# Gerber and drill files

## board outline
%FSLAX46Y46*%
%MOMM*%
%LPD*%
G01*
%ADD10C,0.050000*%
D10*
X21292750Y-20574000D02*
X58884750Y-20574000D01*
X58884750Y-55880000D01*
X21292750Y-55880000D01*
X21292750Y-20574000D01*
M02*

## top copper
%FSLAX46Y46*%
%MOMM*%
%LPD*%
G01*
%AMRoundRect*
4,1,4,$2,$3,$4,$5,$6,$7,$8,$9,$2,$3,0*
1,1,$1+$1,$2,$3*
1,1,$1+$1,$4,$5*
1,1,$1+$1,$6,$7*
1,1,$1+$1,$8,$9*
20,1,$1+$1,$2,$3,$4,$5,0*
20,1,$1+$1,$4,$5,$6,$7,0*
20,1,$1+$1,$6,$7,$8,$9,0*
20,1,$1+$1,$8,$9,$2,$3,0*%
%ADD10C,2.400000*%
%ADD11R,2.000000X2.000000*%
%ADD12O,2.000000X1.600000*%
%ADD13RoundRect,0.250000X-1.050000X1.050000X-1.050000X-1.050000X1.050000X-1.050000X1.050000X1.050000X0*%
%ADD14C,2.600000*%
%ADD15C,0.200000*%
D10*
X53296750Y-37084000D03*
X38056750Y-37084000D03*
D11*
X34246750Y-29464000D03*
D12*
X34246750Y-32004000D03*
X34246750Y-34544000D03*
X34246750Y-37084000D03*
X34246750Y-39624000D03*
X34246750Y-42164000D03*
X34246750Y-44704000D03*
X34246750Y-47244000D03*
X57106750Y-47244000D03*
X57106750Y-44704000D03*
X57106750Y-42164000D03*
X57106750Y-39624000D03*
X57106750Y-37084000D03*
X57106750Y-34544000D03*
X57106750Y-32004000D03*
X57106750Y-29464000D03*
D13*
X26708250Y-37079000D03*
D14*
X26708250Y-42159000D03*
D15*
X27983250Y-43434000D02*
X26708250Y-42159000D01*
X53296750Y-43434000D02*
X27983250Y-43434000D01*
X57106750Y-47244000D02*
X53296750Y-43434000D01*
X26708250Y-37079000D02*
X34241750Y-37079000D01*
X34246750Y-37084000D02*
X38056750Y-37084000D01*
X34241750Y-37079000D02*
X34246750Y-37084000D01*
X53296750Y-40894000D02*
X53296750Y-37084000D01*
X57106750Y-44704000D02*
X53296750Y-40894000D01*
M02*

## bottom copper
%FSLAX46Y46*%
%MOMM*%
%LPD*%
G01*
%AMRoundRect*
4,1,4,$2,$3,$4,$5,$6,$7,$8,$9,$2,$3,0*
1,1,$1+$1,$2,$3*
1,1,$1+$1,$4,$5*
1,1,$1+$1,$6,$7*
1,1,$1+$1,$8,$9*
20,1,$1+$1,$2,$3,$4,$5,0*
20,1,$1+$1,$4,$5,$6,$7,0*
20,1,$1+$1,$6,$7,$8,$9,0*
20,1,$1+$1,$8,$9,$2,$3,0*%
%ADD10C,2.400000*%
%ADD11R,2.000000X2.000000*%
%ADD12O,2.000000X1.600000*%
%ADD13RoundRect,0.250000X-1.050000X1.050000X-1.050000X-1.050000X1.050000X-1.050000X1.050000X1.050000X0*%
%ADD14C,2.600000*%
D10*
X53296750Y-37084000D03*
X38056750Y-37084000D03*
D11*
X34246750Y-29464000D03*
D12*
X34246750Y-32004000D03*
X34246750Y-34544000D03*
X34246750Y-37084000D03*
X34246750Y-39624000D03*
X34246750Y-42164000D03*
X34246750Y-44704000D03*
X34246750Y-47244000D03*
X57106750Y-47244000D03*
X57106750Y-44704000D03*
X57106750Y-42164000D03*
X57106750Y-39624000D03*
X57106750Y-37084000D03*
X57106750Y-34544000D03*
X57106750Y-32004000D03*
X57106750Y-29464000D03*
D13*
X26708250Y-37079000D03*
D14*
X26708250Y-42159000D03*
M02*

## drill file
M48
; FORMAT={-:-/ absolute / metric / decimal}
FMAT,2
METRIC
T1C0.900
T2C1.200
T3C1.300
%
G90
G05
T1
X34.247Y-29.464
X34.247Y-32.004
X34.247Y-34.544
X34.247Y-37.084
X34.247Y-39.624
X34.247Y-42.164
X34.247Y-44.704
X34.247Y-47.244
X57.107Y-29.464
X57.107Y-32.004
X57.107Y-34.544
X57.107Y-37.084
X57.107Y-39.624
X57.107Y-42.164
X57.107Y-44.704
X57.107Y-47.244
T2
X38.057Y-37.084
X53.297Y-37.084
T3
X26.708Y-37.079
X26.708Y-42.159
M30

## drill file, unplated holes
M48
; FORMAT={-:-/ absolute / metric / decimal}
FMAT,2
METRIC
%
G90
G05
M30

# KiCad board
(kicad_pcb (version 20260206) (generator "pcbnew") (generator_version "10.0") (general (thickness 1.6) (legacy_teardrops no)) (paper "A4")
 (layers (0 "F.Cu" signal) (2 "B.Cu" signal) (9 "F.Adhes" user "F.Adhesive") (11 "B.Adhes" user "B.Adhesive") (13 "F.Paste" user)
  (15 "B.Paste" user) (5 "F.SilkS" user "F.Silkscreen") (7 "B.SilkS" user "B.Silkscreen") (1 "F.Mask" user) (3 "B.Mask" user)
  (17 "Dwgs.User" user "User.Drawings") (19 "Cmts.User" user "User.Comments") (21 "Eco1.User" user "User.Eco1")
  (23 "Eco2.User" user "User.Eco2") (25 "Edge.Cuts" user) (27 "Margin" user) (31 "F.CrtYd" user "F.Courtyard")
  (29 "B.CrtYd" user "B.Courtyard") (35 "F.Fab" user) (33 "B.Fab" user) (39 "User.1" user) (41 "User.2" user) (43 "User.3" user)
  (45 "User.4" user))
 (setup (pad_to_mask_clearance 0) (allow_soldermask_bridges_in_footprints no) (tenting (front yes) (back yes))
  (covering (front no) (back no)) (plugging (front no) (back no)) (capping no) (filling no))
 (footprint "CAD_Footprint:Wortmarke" (layer "F.Cu") (at 26.924 47.498)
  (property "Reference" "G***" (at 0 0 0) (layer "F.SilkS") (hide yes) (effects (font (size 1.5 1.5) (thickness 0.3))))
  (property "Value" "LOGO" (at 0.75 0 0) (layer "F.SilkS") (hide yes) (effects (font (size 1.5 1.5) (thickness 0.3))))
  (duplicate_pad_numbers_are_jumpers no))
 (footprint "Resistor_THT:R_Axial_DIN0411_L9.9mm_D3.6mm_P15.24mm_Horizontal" (layer "F.Cu") (at 53.29675 37.084 180)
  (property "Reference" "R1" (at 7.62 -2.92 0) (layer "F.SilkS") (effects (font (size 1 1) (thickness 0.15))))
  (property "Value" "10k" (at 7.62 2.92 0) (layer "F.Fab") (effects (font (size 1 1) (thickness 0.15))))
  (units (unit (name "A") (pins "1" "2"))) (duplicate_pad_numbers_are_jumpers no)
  (pad "1" thru_hole circle (at 0 0 180) (size 2.4 2.4) (drill 1.2) (layers "*.Cu" "*.Mask") (remove_unused_layers no) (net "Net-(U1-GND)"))
  (pad "2" thru_hole circle (at 15.24 0 180) (size 2.4 2.4) (drill 1.2) (layers "*.Cu" "*.Mask") (remove_unused_layers no)
   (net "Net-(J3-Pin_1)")))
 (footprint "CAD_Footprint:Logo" (layer "F.Cu") (at 26.924 27.432)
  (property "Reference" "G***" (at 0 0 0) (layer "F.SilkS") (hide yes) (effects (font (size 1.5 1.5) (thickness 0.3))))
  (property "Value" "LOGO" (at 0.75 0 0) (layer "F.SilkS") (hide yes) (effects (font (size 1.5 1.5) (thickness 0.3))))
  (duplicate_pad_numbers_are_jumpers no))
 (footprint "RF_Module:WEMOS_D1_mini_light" (layer "F.Cu") (at 34.24675 29.464)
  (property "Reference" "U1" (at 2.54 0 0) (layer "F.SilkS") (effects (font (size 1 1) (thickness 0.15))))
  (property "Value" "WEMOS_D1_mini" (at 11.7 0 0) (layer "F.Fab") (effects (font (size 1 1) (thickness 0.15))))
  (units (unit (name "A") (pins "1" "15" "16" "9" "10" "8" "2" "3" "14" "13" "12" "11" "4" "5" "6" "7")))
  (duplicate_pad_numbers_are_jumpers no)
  (pad "1" thru_hole rect (at 0 0) (size 2 2) (drill 0.9) (layers "*.Cu" "*.Mask") (remove_unused_layers no)
   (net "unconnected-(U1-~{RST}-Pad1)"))
  (pad "2" thru_hole oval (at 0 2.54) (size 2 1.6) (drill 0.9) (layers "*.Cu" "*.Mask") (remove_unused_layers no)
   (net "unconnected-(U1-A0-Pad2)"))
  (pad "3" thru_hole oval (at 0 5.08) (size 2 1.6) (drill 0.9) (layers "*.Cu" "*.Mask") (remove_unused_layers no)
   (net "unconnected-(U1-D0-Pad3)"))
  (pad "4" thru_hole oval (at 0 7.62) (size 2 1.6) (drill 0.9) (layers "*.Cu" "*.Mask") (remove_unused_layers no) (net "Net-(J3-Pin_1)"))
  (pad "5" thru_hole oval (at 0 10.16) (size 2 1.6) (drill 0.9) (layers "*.Cu" "*.Mask") (remove_unused_layers no)
   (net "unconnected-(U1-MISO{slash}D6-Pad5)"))
  (pad "6" thru_hole oval (at 0 12.7) (size 2 1.6) (drill 0.9) (layers "*.Cu" "*.Mask") (remove_unused_layers no)
   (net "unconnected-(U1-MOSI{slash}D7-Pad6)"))
  (pad "7" thru_hole oval (at 0 15.24) (size 2 1.6) (drill 0.9) (layers "*.Cu" "*.Mask") (remove_unused_layers no)
   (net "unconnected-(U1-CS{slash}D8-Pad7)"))
  (pad "8" thru_hole oval (at 0 17.78) (size 2 1.6) (drill 0.9) (layers "*.Cu" "*.Mask") (remove_unused_layers no)
   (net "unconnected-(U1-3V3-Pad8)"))
  (pad "9" thru_hole oval (at 22.86 17.78) (size 2 1.6) (drill 0.9) (layers "*.Cu" "*.Mask") (remove_unused_layers no)
   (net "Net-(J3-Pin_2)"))
  (pad "10" thru_hole oval (at 22.86 15.24) (size 2 1.6) (drill 0.9) (layers "*.Cu" "*.Mask") (remove_unused_layers no) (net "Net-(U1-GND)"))
  (pad "11" thru_hole oval (at 22.86 12.7) (size 2 1.6) (drill 0.9) (layers "*.Cu" "*.Mask") (remove_unused_layers no)
   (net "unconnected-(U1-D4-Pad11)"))
  (pad "12" thru_hole oval (at 22.86 10.16) (size 2 1.6) (drill 0.9) (layers "*.Cu" "*.Mask") (remove_unused_layers no)
   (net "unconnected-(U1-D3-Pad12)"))
  (pad "13" thru_hole oval (at 22.86 7.62) (size 2 1.6) (drill 0.9) (layers "*.Cu" "*.Mask") (remove_unused_layers no)
   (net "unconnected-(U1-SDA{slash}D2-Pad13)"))
  (pad "14" thru_hole oval (at 22.86 5.08) (size 2 1.6) (drill 0.9) (layers "*.Cu" "*.Mask") (remove_unused_layers no)
   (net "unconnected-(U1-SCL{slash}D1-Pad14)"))
  (pad "15" thru_hole oval (at 22.86 2.54) (size 2 1.6) (drill 0.9) (layers "*.Cu" "*.Mask") (remove_unused_layers no)
   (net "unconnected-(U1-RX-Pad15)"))
  (pad "16" thru_hole oval (at 22.86 0) (size 2 1.6) (drill 0.9) (layers "*.Cu" "*.Mask") (remove_unused_layers no)
   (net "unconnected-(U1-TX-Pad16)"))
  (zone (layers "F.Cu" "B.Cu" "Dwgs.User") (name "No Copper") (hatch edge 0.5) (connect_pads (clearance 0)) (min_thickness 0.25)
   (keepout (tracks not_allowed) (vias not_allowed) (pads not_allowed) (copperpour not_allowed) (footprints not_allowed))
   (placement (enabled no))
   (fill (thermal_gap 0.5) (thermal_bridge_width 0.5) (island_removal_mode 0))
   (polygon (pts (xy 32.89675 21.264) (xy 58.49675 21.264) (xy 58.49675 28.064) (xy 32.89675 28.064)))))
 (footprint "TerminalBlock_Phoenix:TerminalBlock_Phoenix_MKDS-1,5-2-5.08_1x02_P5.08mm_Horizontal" (layer "F.Cu") (at 26.70825 37.079 -90)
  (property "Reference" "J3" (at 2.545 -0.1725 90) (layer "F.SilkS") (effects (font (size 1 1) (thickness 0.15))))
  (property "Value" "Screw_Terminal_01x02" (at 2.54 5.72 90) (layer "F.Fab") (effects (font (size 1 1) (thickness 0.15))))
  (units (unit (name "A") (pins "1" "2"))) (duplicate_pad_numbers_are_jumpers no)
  (pad "1" thru_hole roundrect (at 0 0 270) (size 2.6 2.6) (drill 1.3) (layers "*.Cu" "*.Mask") (remove_unused_layers no)
   (roundrect_rratio 0.096154) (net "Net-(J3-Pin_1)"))
  (pad "2" thru_hole circle (at 5.08 0 270) (size 2.6 2.6) (drill 1.3) (layers "*.Cu" "*.Mask") (remove_unused_layers no)
   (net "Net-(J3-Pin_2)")))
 (gr_rect (start 21.29275 20.574) (end 58.88475 55.88) (stroke (width 0.05) (type default)) (fill no) (layer "Edge.Cuts"))
 (segment (start 53.29675 40.894) (end 53.29675 37.084) (width 0.2) (layer "F.Cu") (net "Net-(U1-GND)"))
 (segment (start 57.10675 44.704) (end 53.29675 40.894) (width 0.2) (layer "F.Cu") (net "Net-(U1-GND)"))
 (segment (start 26.70825 37.079) (end 34.24175 37.079) (width 0.2) (layer "F.Cu") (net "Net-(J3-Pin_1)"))
 (segment (start 34.24675 37.084) (end 38.05675 37.084) (width 0.2) (layer "F.Cu") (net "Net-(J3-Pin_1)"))
 (segment (start 34.24175 37.079) (end 34.24675 37.084) (width 0.2) (layer "F.Cu") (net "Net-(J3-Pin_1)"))
 (segment (start 27.98325 43.434) (end 26.70825 42.159) (width 0.2) (layer "F.Cu") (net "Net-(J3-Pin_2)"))
 (segment (start 53.29675 43.434) (end 27.98325 43.434) (width 0.2) (layer "F.Cu") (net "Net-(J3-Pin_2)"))
 (segment (start 57.10675 47.244) (end 53.29675 43.434) (width 0.2) (layer "F.Cu") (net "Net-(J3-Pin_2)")))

